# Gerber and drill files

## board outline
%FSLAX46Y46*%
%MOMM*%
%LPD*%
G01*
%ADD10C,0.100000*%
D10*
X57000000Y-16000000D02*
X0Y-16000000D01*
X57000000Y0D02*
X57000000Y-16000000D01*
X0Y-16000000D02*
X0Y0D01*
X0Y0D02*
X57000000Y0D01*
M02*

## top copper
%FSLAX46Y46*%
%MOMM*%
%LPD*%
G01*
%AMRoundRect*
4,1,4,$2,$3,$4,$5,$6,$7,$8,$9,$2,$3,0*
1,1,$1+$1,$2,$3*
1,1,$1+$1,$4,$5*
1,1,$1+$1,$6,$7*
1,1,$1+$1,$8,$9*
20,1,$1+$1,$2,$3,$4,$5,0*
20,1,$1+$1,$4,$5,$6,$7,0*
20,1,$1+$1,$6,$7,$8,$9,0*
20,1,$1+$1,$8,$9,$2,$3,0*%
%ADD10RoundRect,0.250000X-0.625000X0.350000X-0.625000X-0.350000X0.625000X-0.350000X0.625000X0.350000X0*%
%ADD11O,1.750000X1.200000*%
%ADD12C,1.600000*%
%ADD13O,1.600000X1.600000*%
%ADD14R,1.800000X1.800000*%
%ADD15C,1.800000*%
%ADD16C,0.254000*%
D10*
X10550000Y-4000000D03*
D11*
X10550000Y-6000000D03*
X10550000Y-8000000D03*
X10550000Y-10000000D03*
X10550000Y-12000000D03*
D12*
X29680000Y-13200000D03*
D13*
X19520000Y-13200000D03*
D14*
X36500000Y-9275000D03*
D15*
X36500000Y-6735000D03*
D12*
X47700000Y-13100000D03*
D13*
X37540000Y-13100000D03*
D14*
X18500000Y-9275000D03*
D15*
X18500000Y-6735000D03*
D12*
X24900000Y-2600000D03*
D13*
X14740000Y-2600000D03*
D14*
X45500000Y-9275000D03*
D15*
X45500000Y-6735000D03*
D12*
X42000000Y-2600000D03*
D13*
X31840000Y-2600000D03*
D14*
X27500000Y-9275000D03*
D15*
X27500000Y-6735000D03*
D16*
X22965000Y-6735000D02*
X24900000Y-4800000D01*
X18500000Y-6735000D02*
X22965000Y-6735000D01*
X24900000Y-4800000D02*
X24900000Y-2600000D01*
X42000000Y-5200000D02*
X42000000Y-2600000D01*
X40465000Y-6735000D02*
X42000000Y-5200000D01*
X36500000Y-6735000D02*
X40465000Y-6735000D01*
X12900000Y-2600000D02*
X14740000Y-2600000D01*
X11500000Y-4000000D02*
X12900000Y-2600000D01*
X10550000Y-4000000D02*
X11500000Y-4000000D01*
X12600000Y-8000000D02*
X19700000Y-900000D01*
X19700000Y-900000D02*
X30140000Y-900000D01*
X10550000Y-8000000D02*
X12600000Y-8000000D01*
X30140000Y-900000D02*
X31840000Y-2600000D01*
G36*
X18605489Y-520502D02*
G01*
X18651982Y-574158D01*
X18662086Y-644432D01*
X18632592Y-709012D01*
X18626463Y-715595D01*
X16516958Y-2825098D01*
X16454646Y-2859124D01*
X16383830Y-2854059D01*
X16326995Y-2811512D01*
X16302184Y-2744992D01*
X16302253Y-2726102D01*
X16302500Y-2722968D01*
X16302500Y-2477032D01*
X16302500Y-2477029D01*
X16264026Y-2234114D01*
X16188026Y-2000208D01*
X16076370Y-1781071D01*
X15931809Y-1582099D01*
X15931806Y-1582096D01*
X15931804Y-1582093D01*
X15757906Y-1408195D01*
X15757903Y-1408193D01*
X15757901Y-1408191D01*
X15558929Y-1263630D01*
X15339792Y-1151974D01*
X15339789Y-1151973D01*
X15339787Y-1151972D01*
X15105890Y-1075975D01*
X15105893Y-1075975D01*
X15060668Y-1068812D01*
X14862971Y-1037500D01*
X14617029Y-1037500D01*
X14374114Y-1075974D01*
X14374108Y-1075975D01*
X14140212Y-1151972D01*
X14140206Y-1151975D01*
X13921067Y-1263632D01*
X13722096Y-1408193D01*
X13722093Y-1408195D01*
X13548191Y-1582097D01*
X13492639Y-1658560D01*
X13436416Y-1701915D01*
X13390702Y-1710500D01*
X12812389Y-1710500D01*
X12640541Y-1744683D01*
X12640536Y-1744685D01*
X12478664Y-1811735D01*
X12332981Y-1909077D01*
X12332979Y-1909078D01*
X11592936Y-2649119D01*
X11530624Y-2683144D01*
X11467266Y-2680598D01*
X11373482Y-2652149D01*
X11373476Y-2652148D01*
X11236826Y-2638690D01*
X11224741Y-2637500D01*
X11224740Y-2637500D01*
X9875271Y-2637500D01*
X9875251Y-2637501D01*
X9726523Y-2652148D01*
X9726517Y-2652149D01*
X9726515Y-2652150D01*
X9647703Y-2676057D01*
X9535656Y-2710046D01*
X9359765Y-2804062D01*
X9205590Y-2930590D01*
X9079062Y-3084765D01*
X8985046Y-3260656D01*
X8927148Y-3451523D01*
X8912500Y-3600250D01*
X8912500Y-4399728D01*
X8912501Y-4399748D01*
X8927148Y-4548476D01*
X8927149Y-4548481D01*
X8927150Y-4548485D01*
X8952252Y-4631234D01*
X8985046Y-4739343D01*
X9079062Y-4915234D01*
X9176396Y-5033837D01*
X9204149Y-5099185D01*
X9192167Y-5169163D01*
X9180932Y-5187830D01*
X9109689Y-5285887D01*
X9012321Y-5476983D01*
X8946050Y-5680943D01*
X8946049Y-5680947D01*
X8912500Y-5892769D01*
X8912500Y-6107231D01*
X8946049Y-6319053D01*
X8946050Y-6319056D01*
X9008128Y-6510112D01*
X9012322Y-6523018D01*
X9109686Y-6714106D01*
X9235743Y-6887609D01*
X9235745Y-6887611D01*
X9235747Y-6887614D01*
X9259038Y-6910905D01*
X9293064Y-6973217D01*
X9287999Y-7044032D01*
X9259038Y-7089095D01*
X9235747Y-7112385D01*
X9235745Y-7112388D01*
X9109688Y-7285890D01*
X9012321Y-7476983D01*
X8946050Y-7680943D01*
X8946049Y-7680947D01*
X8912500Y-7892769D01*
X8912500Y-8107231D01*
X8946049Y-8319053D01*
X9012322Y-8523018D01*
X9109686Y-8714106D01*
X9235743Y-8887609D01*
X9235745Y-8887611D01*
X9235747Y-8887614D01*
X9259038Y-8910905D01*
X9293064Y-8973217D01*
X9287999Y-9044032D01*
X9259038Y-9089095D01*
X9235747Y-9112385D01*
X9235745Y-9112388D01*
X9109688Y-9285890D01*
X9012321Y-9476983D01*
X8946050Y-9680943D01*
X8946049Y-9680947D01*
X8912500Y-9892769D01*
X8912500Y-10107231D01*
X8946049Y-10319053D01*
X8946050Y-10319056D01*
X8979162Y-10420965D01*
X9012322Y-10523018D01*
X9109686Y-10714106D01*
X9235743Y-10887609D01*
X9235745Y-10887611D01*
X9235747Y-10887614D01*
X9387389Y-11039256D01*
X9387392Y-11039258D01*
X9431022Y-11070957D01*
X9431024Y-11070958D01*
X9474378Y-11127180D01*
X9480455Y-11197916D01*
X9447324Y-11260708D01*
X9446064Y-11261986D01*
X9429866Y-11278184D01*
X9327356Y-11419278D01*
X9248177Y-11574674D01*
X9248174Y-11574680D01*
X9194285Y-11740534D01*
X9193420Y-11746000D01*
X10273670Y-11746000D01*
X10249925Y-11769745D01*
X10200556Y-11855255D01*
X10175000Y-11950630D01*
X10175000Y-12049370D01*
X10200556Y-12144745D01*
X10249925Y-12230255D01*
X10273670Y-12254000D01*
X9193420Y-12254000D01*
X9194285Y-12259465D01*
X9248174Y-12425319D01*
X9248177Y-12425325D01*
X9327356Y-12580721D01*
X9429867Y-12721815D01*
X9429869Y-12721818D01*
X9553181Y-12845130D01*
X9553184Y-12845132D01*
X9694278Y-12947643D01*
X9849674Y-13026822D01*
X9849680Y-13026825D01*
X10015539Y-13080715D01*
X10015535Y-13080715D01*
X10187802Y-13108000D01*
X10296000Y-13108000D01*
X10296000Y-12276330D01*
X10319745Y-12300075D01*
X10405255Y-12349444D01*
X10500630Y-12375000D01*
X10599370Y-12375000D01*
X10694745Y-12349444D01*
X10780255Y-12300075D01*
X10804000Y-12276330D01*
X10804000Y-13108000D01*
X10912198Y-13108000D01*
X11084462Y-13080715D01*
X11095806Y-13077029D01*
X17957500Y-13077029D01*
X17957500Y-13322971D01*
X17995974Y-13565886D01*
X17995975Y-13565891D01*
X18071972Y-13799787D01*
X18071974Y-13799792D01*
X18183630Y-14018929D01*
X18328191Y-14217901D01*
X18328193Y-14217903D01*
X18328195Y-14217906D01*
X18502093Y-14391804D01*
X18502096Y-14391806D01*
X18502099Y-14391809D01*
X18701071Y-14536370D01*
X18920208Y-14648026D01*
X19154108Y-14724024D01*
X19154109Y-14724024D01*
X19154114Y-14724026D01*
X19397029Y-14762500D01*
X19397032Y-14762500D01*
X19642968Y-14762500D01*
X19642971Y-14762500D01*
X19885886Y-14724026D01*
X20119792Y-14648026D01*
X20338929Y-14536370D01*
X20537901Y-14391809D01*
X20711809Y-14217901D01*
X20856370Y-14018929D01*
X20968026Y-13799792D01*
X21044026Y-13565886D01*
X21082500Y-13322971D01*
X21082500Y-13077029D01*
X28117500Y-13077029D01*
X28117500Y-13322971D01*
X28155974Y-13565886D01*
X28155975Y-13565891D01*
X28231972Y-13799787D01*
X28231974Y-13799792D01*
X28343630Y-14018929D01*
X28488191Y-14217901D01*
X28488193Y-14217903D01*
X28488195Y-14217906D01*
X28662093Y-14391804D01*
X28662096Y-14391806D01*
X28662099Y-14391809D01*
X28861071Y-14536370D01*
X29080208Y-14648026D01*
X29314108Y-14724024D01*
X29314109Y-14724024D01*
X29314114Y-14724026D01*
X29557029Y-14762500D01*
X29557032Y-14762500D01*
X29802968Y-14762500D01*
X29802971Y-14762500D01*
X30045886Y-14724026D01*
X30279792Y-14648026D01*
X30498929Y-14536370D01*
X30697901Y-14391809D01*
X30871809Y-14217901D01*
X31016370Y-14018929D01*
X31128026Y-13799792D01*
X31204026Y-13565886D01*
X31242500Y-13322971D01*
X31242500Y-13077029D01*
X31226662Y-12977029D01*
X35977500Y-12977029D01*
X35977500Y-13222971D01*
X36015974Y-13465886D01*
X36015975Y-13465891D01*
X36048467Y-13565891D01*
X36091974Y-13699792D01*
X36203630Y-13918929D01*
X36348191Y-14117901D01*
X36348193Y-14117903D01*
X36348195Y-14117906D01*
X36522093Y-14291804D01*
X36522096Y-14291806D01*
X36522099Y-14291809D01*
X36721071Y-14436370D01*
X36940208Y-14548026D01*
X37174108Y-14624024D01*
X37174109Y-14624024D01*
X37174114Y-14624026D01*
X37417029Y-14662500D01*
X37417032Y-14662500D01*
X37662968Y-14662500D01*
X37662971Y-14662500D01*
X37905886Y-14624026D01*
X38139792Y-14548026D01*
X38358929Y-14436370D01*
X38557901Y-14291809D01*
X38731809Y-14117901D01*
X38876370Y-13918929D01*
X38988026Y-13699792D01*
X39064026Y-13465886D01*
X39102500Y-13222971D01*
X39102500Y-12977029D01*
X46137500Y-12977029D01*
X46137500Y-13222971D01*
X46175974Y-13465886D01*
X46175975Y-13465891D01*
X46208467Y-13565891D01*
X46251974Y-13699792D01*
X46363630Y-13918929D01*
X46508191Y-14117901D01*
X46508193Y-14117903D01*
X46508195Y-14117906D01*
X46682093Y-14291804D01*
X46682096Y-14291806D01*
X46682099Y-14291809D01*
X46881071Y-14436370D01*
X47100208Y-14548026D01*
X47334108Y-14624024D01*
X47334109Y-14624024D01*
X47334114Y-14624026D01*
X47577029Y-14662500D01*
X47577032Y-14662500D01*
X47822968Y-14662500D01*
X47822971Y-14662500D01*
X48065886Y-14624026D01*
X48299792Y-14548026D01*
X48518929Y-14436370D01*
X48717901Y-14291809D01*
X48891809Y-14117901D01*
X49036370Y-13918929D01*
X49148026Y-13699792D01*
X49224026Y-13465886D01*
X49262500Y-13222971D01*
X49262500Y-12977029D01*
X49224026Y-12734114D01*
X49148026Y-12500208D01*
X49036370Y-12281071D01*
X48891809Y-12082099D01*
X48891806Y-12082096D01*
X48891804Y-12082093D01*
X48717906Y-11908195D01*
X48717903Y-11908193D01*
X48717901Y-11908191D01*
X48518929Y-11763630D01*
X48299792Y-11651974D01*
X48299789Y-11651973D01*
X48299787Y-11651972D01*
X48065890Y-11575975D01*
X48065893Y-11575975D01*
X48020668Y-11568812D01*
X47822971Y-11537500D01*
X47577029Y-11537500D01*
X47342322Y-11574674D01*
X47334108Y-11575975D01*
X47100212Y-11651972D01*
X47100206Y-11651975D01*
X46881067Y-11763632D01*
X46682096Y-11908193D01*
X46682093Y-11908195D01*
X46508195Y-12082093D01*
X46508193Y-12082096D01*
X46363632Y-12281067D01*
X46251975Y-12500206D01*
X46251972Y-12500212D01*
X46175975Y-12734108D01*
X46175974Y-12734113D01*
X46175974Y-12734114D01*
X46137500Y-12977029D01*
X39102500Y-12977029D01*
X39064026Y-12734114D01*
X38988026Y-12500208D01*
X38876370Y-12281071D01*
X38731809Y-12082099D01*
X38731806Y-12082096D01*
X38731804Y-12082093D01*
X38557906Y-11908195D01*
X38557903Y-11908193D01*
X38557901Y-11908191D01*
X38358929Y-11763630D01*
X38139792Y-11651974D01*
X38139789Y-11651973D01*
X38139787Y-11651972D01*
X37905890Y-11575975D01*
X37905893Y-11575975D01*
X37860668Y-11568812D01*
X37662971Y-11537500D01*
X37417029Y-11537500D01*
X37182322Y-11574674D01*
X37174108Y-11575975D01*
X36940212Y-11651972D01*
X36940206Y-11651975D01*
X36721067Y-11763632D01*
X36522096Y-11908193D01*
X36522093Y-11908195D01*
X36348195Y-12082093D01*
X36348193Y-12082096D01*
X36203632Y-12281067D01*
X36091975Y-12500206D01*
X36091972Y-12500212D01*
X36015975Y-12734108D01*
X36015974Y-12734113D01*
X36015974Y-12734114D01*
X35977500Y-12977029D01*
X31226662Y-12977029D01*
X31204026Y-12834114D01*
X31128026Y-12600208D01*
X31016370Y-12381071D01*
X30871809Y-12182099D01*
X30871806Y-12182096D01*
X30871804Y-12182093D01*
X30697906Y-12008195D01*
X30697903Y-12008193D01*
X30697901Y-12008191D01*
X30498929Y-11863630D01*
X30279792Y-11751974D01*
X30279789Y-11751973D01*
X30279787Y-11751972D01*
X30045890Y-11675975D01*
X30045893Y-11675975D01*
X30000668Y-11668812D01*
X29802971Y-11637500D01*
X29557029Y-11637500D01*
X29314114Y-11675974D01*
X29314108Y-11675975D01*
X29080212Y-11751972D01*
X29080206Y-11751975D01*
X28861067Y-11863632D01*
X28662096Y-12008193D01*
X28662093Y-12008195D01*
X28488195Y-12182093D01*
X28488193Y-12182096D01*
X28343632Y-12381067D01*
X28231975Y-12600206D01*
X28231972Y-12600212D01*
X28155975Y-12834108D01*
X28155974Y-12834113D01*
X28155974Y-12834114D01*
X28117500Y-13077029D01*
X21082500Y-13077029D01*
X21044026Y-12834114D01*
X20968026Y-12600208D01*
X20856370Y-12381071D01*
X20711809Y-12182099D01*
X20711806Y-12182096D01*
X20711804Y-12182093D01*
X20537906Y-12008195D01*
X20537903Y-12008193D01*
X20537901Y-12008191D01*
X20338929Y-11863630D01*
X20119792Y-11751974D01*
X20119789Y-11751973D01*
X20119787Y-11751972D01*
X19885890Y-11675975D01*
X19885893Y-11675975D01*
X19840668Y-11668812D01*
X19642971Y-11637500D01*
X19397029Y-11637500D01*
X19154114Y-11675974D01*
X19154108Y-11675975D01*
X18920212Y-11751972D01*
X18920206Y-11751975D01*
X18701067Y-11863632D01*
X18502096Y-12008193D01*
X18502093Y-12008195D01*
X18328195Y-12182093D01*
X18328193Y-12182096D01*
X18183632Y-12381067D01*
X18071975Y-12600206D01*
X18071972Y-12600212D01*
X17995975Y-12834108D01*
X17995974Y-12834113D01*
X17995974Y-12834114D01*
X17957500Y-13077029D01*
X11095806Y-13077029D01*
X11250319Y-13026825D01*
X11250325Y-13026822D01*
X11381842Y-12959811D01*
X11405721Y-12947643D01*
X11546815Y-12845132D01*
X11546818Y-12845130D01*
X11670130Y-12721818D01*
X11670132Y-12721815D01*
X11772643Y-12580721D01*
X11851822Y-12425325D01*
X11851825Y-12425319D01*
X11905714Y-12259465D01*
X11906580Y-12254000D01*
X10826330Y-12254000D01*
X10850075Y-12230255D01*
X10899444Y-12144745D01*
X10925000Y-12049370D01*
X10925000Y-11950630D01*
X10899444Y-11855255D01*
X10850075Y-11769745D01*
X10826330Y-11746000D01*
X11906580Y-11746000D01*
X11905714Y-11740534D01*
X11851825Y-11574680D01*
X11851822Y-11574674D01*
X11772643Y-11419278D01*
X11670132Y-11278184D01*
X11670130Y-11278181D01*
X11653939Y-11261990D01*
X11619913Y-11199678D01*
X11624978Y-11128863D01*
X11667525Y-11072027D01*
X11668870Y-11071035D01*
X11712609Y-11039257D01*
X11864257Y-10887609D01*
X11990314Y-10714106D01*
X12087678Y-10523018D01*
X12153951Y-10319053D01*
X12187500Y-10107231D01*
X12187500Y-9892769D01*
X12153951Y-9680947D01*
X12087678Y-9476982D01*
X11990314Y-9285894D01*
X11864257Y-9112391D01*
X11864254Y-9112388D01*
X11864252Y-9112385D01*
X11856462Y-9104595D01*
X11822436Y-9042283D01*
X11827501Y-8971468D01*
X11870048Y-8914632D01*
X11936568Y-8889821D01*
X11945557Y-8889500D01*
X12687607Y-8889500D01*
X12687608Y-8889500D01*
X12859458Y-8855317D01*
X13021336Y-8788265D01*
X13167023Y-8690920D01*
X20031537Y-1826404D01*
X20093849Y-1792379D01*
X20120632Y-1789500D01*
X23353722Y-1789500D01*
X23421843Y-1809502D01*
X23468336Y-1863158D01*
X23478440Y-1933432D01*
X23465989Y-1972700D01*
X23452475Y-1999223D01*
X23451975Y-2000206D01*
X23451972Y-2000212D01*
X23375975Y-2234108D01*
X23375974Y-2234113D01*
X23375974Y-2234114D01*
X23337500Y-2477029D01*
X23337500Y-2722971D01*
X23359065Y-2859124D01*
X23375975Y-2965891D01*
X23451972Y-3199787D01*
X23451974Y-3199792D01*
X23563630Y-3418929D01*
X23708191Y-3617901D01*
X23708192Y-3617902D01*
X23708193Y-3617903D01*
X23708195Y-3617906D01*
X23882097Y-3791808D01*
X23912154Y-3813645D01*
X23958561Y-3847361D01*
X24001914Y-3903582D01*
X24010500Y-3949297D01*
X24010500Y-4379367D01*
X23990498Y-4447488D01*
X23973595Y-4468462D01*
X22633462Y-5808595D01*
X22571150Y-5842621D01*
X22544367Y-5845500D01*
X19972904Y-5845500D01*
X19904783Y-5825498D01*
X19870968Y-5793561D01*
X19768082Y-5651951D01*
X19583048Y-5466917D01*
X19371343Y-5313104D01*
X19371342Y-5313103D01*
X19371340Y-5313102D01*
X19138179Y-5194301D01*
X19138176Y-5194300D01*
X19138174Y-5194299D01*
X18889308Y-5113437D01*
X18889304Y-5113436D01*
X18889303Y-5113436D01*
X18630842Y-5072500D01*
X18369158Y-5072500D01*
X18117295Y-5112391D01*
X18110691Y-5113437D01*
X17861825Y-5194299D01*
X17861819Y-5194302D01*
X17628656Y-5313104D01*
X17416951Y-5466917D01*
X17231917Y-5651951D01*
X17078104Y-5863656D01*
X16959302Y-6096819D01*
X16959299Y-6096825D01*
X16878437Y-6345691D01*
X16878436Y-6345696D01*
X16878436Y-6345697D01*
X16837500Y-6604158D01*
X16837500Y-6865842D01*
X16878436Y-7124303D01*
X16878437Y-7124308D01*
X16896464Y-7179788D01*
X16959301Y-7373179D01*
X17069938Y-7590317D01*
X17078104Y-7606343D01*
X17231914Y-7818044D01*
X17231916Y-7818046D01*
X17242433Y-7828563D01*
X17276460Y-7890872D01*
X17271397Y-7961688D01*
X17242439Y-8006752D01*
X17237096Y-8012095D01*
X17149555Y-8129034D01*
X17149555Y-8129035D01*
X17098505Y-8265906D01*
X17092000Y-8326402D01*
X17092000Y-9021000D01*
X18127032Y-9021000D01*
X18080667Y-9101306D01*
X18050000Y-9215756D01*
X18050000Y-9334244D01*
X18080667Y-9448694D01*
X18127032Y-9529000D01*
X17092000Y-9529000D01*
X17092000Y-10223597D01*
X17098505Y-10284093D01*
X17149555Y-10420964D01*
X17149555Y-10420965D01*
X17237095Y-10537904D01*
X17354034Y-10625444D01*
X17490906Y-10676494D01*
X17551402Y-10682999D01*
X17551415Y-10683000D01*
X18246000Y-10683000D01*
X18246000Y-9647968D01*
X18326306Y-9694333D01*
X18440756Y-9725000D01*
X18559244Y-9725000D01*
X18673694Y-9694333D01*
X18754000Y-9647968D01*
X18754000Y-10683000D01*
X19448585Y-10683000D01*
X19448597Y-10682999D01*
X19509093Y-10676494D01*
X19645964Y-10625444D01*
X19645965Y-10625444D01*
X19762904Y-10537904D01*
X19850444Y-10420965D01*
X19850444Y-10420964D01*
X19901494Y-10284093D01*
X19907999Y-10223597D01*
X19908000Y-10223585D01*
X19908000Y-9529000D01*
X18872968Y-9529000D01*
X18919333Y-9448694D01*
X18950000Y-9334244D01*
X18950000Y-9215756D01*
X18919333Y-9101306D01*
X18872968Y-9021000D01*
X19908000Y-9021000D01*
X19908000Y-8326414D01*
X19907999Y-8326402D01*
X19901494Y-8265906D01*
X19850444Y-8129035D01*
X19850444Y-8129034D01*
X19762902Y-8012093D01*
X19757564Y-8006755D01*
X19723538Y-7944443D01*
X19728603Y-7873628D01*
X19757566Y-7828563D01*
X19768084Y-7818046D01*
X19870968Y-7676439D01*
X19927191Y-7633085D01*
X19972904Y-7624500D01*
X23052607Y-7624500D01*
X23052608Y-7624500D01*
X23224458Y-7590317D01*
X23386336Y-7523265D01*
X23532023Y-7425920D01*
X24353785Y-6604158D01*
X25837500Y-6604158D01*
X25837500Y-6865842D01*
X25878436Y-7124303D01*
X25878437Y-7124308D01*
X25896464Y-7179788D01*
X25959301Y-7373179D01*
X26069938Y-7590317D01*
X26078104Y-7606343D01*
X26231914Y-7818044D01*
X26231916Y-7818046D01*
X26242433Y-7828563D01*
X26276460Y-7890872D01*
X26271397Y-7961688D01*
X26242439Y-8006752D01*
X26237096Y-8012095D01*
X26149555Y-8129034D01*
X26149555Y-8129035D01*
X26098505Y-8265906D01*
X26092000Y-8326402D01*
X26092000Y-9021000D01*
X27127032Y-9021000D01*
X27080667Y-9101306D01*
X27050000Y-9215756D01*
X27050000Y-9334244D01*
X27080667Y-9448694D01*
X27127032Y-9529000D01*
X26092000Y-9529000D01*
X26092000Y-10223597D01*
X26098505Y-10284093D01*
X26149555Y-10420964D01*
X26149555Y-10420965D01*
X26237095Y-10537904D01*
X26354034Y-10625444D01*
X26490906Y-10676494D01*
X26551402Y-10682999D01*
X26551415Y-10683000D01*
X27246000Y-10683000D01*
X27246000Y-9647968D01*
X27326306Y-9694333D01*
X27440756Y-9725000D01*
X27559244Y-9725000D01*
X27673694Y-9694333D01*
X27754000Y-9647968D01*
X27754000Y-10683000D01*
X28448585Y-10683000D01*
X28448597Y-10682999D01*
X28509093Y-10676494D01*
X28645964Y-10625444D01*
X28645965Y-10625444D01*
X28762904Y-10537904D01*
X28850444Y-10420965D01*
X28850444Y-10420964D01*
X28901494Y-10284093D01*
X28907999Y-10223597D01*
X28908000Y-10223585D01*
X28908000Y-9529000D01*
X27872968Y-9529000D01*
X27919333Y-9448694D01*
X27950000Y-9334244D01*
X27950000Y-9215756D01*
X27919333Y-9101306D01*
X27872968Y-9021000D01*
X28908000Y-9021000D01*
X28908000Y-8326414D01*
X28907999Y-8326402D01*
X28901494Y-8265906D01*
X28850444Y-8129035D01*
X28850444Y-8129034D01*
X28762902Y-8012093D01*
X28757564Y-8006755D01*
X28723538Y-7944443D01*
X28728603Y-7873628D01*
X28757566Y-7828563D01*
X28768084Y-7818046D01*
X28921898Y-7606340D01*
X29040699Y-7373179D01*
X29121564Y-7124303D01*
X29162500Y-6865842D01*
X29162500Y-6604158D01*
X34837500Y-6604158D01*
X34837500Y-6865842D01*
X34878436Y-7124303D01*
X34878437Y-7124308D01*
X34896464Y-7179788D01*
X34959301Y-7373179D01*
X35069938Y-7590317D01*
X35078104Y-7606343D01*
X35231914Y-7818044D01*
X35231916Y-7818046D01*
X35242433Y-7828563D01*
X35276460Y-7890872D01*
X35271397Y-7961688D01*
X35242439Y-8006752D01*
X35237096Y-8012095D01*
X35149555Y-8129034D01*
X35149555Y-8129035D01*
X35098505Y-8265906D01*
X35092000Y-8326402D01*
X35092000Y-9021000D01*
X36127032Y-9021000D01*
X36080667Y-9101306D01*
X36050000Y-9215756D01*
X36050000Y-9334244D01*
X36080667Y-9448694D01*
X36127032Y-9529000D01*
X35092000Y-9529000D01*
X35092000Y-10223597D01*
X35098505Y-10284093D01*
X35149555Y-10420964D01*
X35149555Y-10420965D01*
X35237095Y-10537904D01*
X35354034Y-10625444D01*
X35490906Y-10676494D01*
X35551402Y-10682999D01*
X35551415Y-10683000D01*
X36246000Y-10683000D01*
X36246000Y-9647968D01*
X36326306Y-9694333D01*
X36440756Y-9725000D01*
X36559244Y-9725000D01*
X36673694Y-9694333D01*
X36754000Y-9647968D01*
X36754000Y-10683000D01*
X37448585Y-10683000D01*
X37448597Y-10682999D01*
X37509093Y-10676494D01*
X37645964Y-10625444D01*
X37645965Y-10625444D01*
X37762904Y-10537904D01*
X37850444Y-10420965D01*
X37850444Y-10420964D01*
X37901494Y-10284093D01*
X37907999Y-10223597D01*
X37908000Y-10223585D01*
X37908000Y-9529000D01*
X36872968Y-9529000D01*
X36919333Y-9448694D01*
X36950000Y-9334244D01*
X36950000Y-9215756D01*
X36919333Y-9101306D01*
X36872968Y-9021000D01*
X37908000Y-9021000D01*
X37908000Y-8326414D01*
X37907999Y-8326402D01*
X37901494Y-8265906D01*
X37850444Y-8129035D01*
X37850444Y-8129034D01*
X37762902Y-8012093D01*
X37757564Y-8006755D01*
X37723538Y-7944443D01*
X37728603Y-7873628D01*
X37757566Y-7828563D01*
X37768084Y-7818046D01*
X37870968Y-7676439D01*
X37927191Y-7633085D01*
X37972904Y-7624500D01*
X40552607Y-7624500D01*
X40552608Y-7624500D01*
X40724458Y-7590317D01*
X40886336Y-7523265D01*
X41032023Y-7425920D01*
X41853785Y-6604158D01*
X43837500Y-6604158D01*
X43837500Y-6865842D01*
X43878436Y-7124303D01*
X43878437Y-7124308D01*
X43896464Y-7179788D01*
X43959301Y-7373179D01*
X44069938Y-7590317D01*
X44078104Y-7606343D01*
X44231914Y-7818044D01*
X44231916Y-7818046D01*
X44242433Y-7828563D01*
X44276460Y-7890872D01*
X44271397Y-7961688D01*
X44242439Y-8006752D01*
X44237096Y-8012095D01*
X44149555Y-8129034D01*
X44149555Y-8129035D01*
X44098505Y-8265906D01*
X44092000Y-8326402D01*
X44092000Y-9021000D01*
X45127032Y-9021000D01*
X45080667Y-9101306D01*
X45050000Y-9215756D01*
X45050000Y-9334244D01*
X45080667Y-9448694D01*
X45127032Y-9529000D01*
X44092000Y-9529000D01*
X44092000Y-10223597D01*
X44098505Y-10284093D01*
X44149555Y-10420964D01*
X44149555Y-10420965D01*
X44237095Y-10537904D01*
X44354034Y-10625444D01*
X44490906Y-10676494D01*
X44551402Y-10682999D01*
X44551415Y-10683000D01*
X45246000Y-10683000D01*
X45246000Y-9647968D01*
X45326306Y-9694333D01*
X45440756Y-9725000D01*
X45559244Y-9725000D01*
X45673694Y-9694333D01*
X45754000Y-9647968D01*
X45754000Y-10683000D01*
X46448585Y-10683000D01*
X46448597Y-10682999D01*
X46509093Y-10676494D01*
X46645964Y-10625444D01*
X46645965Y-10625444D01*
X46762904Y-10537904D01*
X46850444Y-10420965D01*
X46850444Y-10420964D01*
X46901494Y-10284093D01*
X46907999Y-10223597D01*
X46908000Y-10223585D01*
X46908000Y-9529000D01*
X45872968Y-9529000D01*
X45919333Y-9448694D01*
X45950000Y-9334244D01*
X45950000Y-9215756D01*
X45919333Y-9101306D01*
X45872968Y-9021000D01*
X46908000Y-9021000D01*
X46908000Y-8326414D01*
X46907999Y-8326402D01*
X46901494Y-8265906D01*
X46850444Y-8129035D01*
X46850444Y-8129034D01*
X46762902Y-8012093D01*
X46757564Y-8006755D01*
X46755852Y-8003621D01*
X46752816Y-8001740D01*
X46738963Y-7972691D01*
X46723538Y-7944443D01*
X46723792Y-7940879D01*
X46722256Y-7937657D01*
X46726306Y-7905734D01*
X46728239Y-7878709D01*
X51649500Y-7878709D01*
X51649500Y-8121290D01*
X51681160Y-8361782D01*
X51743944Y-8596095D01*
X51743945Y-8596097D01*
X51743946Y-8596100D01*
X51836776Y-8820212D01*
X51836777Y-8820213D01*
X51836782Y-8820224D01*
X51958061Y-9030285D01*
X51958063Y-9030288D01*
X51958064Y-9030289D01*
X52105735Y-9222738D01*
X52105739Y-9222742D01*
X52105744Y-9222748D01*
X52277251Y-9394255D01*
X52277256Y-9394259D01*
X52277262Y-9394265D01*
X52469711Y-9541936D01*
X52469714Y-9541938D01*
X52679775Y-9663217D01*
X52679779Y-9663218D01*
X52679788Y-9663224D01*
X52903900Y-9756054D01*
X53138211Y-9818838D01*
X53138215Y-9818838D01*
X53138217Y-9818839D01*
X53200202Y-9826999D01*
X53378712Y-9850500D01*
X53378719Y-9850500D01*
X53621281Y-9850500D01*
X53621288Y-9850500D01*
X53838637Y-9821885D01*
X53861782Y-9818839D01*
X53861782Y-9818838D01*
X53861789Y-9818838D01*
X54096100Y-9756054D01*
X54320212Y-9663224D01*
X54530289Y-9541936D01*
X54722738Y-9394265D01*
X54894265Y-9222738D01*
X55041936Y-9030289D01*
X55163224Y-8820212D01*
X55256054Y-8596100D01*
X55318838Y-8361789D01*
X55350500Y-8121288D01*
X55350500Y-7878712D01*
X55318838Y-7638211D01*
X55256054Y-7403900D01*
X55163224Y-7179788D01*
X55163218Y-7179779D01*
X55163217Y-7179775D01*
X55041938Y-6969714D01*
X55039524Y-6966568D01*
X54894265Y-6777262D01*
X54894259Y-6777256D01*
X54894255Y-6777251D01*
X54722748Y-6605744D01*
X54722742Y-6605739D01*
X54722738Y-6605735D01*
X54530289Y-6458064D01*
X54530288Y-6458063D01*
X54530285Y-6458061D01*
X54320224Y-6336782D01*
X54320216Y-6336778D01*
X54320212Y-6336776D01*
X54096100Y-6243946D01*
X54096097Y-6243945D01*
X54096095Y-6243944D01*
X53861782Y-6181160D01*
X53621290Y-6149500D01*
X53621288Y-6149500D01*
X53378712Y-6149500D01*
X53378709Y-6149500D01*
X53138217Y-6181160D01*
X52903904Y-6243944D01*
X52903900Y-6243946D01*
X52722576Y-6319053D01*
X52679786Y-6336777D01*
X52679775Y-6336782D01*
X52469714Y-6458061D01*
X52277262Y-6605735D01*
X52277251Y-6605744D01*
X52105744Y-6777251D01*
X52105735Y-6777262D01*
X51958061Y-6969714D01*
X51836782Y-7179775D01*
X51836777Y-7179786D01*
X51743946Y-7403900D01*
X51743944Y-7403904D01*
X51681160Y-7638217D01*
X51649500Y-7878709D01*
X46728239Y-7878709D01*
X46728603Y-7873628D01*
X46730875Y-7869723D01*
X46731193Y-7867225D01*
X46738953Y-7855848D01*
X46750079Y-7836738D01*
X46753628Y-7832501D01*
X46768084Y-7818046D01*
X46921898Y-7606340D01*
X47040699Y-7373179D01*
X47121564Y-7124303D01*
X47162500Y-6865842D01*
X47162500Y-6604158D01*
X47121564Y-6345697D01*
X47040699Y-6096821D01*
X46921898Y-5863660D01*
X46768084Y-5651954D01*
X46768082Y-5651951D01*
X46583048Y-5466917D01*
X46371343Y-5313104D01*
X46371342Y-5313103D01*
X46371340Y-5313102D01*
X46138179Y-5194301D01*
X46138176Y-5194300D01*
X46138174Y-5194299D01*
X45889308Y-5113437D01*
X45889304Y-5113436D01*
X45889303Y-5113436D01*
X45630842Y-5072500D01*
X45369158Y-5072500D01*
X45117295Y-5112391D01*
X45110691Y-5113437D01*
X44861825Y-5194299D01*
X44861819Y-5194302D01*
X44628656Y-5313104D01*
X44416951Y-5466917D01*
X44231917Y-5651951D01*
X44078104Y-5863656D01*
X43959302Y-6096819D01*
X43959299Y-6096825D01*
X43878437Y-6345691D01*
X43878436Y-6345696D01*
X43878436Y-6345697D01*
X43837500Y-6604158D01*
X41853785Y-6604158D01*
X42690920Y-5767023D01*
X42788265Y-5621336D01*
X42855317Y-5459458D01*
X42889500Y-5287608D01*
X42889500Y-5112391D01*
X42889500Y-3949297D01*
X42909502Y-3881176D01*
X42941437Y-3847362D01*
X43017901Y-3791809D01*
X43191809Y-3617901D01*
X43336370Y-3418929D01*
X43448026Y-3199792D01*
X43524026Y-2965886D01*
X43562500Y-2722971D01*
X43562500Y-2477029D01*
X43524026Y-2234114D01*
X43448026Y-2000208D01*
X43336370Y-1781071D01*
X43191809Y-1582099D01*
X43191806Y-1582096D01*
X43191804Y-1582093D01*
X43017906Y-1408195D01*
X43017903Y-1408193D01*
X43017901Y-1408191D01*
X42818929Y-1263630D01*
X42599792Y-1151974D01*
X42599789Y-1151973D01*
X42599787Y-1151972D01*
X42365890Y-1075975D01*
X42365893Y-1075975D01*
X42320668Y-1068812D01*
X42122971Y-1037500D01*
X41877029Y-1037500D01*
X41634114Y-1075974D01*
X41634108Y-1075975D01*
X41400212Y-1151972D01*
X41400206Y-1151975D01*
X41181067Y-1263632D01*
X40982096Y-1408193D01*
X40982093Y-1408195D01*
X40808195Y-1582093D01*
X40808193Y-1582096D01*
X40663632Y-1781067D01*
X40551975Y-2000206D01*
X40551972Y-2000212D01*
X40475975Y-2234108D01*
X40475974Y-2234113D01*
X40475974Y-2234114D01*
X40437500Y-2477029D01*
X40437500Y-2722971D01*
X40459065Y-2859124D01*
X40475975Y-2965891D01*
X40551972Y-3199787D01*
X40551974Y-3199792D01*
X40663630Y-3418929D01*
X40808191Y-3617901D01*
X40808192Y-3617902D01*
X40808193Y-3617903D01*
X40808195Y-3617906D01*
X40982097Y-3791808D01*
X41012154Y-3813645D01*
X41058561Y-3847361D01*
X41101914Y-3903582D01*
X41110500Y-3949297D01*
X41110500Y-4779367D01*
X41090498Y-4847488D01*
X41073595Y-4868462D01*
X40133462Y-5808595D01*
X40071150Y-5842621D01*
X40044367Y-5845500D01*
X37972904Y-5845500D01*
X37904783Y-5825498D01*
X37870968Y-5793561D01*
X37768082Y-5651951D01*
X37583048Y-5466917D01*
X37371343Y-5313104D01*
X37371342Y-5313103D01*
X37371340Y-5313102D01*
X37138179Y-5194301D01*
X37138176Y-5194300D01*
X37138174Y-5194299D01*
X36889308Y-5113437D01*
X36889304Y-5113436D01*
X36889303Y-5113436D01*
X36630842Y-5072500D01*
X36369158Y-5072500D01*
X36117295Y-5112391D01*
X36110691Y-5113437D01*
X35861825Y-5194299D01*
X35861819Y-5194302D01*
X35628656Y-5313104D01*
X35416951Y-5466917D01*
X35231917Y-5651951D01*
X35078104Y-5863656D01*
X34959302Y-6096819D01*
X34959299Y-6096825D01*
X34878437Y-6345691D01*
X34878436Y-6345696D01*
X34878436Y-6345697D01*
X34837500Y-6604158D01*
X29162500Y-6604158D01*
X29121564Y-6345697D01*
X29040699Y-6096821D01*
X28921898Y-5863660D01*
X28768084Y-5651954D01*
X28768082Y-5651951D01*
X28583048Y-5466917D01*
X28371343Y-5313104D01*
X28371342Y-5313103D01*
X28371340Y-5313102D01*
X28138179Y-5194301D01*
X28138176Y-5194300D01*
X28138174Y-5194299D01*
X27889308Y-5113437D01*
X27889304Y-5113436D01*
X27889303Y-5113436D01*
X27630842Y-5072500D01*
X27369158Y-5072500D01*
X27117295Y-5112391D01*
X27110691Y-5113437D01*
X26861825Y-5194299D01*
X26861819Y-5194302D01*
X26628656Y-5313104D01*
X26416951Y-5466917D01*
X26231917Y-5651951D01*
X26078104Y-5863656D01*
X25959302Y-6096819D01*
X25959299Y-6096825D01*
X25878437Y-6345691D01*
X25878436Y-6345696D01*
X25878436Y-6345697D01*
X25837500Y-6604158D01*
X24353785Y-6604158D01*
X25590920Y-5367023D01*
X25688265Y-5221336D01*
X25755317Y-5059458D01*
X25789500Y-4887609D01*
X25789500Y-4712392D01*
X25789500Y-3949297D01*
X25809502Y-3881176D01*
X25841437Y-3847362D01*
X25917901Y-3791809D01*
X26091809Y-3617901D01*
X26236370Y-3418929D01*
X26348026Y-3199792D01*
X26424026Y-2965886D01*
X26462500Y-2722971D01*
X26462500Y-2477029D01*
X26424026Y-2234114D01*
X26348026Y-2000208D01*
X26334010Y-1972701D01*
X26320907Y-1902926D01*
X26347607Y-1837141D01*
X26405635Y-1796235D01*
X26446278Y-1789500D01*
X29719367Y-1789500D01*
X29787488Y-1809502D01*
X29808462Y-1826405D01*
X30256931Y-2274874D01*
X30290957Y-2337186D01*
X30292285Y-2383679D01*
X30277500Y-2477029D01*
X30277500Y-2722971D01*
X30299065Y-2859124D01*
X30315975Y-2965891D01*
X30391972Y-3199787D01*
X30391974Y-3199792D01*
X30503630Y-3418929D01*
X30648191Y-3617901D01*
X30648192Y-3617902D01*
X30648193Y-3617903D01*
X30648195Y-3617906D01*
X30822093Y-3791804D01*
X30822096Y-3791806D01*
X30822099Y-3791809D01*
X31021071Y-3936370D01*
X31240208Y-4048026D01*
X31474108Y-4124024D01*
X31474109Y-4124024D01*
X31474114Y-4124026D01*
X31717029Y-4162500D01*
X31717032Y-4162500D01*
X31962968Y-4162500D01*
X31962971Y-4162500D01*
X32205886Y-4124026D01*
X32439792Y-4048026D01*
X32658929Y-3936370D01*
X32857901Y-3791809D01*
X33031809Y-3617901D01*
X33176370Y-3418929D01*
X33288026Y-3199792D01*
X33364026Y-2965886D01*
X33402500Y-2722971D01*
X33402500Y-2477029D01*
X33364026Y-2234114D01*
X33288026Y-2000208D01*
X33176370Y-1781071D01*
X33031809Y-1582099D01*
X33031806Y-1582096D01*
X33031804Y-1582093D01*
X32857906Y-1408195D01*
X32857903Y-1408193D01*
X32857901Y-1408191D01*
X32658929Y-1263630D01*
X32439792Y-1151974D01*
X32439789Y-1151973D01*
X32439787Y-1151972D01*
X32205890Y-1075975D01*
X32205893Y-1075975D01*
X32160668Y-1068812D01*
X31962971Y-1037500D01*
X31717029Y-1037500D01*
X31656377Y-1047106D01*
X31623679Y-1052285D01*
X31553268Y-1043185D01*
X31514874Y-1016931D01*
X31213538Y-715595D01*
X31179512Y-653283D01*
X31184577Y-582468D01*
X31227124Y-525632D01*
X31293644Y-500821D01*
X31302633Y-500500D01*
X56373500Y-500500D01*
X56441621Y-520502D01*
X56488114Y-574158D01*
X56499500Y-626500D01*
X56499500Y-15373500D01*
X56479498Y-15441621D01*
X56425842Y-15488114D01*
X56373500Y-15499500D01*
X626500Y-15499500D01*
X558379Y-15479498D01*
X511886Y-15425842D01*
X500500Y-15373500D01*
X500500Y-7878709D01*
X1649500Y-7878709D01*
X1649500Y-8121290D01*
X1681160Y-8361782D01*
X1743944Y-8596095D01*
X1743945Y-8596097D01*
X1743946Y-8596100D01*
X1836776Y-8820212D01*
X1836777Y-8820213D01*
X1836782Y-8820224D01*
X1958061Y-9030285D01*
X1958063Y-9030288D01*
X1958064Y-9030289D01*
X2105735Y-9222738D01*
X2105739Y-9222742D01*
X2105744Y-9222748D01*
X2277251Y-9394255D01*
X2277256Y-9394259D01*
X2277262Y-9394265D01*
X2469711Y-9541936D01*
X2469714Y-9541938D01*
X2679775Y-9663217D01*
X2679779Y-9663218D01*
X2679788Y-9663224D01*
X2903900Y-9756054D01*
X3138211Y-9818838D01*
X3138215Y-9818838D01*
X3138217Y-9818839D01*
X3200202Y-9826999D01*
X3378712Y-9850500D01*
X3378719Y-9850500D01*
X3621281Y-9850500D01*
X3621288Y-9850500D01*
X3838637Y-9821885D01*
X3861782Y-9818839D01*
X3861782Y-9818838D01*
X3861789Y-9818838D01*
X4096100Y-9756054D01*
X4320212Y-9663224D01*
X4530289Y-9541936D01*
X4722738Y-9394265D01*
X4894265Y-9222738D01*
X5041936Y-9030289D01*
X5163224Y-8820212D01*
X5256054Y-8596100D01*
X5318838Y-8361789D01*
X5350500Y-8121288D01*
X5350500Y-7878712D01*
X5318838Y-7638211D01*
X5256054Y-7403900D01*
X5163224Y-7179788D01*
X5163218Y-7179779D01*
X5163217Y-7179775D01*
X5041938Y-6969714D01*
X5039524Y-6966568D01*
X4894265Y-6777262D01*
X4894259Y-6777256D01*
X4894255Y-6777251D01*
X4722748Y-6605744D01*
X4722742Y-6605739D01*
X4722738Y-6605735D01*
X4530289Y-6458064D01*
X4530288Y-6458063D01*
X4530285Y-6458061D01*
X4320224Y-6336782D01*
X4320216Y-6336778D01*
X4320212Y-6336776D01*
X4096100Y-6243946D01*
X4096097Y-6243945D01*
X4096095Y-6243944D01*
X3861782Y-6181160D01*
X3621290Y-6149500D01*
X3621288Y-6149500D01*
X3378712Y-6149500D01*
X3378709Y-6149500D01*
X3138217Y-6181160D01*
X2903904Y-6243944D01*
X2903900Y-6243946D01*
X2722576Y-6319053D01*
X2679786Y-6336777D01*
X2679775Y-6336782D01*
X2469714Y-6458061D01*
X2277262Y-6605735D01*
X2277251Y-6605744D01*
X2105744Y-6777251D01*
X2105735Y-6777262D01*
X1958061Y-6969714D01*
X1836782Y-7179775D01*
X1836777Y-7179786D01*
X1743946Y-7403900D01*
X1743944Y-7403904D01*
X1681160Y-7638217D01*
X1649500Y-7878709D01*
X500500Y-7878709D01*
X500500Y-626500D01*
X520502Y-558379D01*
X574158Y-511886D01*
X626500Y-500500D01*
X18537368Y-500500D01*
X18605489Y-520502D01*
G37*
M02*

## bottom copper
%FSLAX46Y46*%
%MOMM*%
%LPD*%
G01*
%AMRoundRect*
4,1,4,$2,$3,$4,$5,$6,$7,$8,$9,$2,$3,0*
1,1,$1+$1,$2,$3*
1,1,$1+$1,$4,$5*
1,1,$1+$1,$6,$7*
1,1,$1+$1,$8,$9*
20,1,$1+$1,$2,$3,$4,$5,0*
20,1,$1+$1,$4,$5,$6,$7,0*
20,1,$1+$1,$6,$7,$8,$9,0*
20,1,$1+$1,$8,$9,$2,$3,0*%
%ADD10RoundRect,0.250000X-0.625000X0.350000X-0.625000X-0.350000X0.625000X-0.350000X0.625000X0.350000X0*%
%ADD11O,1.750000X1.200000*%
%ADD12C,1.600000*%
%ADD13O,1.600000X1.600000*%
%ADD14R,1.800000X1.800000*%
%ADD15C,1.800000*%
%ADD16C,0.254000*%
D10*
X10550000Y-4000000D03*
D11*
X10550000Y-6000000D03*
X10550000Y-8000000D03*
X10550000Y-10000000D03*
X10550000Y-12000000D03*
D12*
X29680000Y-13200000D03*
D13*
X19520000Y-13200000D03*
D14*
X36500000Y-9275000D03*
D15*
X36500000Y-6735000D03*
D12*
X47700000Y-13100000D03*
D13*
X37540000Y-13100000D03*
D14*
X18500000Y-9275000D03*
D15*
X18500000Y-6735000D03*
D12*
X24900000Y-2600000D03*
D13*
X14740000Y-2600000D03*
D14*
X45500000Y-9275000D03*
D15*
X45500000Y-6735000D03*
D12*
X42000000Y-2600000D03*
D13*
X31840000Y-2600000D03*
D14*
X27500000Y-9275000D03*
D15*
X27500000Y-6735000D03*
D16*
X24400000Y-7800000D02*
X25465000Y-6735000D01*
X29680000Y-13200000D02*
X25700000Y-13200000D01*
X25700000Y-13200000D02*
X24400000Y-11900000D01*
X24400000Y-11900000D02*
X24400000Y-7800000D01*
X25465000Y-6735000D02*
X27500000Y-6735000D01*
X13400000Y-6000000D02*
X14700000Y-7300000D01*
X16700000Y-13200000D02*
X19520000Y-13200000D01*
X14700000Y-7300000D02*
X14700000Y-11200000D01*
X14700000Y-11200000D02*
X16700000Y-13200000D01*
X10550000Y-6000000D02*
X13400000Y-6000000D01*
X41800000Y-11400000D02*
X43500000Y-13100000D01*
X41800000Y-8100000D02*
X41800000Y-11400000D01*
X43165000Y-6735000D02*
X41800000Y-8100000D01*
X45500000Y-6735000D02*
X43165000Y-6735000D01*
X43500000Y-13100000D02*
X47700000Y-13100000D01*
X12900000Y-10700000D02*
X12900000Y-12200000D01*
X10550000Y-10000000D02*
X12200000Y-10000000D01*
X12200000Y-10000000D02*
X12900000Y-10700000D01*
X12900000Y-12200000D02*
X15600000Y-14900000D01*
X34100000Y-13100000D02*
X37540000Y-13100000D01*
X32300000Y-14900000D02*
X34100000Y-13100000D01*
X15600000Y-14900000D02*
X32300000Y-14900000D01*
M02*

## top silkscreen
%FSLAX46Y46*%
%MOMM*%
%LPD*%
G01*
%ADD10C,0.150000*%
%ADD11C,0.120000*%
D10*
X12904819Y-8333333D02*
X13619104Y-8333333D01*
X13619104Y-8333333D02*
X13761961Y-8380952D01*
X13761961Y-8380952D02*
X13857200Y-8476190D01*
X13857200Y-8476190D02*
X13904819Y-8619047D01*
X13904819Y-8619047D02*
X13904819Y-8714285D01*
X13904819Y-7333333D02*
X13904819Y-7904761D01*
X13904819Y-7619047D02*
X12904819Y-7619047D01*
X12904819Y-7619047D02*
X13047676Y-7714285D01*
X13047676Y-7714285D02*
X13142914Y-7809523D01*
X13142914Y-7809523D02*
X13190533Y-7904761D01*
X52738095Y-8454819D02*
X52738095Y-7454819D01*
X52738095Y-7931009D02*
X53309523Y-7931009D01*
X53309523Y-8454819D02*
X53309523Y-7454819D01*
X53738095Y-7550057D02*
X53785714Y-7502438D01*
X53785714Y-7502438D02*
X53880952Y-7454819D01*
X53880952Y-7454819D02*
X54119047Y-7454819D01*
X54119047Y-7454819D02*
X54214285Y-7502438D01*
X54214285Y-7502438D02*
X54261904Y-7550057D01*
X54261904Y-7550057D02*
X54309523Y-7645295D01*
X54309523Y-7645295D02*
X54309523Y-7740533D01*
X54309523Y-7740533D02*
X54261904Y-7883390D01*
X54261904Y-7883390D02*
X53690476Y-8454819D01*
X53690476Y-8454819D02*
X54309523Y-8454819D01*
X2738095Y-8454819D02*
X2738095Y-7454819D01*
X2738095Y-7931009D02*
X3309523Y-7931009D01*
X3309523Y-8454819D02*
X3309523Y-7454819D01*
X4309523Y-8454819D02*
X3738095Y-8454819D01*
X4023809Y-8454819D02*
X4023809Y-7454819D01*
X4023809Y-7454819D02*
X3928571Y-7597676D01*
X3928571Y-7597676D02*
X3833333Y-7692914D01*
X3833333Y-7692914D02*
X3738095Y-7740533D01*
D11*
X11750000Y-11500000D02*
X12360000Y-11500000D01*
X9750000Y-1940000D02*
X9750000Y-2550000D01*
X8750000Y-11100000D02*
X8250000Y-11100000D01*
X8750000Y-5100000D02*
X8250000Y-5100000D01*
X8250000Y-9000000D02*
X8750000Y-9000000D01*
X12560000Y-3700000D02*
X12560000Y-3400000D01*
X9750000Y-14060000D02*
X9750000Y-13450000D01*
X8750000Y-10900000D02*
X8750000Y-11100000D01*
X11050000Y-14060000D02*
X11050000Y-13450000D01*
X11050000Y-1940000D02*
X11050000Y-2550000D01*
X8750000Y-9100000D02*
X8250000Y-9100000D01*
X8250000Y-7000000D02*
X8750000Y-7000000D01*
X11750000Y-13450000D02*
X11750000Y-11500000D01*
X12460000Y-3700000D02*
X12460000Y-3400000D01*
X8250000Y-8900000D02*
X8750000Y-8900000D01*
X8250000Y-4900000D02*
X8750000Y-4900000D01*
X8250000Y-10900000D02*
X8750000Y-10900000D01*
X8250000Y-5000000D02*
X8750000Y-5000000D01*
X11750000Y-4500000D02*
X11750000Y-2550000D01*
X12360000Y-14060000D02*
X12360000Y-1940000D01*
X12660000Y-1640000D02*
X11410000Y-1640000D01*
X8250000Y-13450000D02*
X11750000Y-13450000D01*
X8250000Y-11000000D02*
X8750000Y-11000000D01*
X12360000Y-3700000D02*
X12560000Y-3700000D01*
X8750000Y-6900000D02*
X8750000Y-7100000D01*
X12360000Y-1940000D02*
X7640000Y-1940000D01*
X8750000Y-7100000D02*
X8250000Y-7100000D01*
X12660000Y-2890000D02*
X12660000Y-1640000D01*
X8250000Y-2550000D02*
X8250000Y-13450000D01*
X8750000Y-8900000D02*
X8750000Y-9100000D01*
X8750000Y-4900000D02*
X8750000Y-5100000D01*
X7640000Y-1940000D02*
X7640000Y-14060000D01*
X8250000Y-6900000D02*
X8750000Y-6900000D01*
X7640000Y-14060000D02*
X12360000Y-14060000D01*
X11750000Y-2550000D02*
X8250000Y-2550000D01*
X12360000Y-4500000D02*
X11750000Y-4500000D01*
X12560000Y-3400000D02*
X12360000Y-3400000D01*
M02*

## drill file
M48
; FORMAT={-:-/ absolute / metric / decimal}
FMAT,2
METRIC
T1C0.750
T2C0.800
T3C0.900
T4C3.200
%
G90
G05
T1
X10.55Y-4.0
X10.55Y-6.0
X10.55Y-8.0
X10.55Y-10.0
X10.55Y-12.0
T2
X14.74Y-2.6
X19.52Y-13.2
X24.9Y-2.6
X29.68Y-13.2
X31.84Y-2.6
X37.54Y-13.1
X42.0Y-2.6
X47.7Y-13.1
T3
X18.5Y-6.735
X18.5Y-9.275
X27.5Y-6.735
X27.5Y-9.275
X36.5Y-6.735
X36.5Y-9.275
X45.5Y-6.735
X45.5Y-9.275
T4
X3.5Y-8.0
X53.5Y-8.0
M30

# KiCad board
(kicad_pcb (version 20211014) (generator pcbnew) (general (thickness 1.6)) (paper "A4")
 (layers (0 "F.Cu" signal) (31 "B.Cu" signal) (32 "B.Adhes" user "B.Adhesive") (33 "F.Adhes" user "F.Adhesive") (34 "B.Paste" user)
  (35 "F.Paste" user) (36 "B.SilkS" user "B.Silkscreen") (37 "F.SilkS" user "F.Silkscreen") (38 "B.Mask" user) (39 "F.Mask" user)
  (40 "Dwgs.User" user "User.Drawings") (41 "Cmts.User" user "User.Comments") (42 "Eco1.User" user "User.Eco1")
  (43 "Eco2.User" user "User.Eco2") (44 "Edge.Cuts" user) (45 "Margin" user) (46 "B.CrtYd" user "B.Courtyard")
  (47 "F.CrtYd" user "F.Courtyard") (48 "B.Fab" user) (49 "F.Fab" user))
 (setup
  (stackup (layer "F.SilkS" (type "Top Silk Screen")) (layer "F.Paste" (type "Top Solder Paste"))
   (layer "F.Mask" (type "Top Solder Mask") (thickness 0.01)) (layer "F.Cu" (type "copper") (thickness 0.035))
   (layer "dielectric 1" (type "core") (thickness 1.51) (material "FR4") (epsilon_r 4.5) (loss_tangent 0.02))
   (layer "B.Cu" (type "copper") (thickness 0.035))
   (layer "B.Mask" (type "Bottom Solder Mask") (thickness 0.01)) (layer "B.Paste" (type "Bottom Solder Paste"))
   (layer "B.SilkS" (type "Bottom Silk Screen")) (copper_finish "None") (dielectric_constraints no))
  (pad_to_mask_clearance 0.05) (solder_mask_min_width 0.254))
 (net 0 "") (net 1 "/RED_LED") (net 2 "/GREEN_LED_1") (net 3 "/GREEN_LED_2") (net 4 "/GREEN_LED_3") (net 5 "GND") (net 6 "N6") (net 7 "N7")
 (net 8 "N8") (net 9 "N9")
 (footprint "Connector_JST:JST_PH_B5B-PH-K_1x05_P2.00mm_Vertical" (layer "F.Cu") (at 10.55 4 -90)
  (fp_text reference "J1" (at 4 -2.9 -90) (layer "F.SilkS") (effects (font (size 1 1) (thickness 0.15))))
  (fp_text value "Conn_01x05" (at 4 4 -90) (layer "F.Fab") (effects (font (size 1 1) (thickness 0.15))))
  (fp_line (start 7.5 -1.2) (end 7.5 -1.81) (layer "F.SilkS") (width 0.12))
  (fp_line (start -2.06 0.8) (end -1.45 0.8) (layer "F.SilkS") (width 0.12))
  (fp_line (start 7.1 1.8) (end 7.1 2.3) (layer "F.SilkS") (width 0.12))
  (fp_line (start 1.1 1.8) (end 1.1 2.3) (layer "F.SilkS") (width 0.12))
  (fp_line (start 5 2.3) (end 5 1.8) (layer "F.SilkS") (width 0.12))
  (fp_line (start -0.3 -2.01) (end -0.6 -2.01) (layer "F.SilkS") (width 0.12))
  (fp_line (start 10.06 0.8) (end 9.45 0.8) (layer "F.SilkS") (width 0.12))
  (fp_line (start 6.9 1.8) (end 7.1 1.8) (layer "F.SilkS") (width 0.12))
  (fp_line (start 10.06 -0.5) (end 9.45 -0.5) (layer "F.SilkS") (width 0.12))
  (fp_line (start -2.06 -0.5) (end -1.45 -0.5) (layer "F.SilkS") (width 0.12))
  (fp_line (start 5.1 1.8) (end 5.1 2.3) (layer "F.SilkS") (width 0.12))
  (fp_line (start 3 2.3) (end 3 1.8) (layer "F.SilkS") (width 0.12))
  (fp_line (start 9.45 -1.2) (end 7.5 -1.2) (layer "F.SilkS") (width 0.12))
  (fp_line (start -0.3 -1.91) (end -0.6 -1.91) (layer "F.SilkS") (width 0.12))
  (fp_line (start 4.9 2.3) (end 4.9 1.8) (layer "F.SilkS") (width 0.12))
  (fp_line (start 0.9 2.3) (end 0.9 1.8) (layer "F.SilkS") (width 0.12))
  (fp_line (start 6.9 2.3) (end 6.9 1.8) (layer "F.SilkS") (width 0.12))
  (fp_line (start 1 2.3) (end 1 1.8) (layer "F.SilkS") (width 0.12))
  (fp_line (start 0.5 -1.2) (end -1.45 -1.2) (layer "F.SilkS") (width 0.12))
  (fp_line (start 10.06 -1.81) (end -2.06 -1.81) (layer "F.SilkS") (width 0.12))
  (fp_line (start -2.36 -2.11) (end -2.36 -0.86) (layer "F.SilkS") (width 0.12))
  (fp_line (start 9.45 2.3) (end 9.45 -1.2) (layer "F.SilkS") (width 0.12))
  (fp_line (start 7 2.3) (end 7 1.8) (layer "F.SilkS") (width 0.12))
  (fp_line (start -0.3 -1.81) (end -0.3 -2.01) (layer "F.SilkS") (width 0.12))
  (fp_line (start 2.9 1.8) (end 3.1 1.8) (layer "F.SilkS") (width 0.12))
  (fp_line (start -2.06 -1.81) (end -2.06 2.91) (layer "F.SilkS") (width 0.12))
  (fp_line (start 3.1 1.8) (end 3.1 2.3) (layer "F.SilkS") (width 0.12))
  (fp_line (start -1.11 -2.11) (end -2.36 -2.11) (layer "F.SilkS") (width 0.12))
  (fp_line (start -1.45 2.3) (end 9.45 2.3) (layer "F.SilkS") (width 0.12))
  (fp_line (start 4.9 1.8) (end 5.1 1.8) (layer "F.SilkS") (width 0.12))
  (fp_line (start 0.9 1.8) (end 1.1 1.8) (layer "F.SilkS") (width 0.12))
  (fp_line (start -2.06 2.91) (end 10.06 2.91) (layer "F.SilkS") (width 0.12))
  (fp_line (start 2.9 2.3) (end 2.9 1.8) (layer "F.SilkS") (width 0.12))
  (fp_line (start 10.06 2.91) (end 10.06 -1.81) (layer "F.SilkS") (width 0.12))
  (fp_line (start -1.45 -1.2) (end -1.45 2.3) (layer "F.SilkS") (width 0.12))
  (fp_line (start 0.5 -1.81) (end 0.5 -1.2) (layer "F.SilkS") (width 0.12))
  (fp_line (start -0.6 -2.01) (end -0.6 -1.81) (layer "F.SilkS") (width 0.12))
  (pad "1" thru_hole roundrect (at 0 0 270) (size 1.2 1.75) (drill 0.75) (layers *.Cu *.Mask) (roundrect_rratio 0.208333) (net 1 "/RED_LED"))
  (pad "2" thru_hole oval (at 2 0 270) (size 1.2 1.75) (drill 0.75) (layers *.Cu *.Mask) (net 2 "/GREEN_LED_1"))
  (pad "3" thru_hole oval (at 4 0 270) (size 1.2 1.75) (drill 0.75) (layers *.Cu *.Mask) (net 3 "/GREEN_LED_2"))
  (pad "4" thru_hole oval (at 6 0 270) (size 1.2 1.75) (drill 0.75) (layers *.Cu *.Mask) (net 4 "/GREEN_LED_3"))
  (pad "5" thru_hole oval (at 8 0 270) (size 1.2 1.75) (drill 0.75) (layers *.Cu *.Mask) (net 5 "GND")))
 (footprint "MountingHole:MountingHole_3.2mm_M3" (layer "F.Cu") (at 53.5 8)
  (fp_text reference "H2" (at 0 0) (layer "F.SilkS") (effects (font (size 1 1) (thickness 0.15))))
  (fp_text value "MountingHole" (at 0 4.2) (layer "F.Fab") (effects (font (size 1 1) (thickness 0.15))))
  (pad "" np_thru_hole circle (at 0 0) (size 3.2 3.2) (drill 3.2) (layers *.Cu *.Mask)))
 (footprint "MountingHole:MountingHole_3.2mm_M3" (layer "F.Cu") (at 3.5 8)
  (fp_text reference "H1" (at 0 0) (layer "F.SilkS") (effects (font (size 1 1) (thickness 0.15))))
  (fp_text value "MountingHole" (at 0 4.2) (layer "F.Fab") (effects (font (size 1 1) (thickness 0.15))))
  (pad "" np_thru_hole circle (at 0 0) (size 3.2 3.2) (drill 3.2) (layers *.Cu *.Mask)))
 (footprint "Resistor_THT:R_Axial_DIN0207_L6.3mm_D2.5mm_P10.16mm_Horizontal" (layer "B.Cu") (at 29.68 13.2 180)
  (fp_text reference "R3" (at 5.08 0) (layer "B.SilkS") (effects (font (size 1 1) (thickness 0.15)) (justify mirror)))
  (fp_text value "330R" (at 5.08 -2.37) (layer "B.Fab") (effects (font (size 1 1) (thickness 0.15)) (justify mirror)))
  (pad "1" thru_hole circle (at 0 0 180) (size 1.6 1.6) (drill 0.8) (layers *.Cu *.Mask) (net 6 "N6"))
  (pad "2" thru_hole oval (at 10.16 0 180) (size 1.6 1.6) (drill 0.8) (layers *.Cu *.Mask) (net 2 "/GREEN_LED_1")))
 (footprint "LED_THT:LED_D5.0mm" (layer "B.Cu") (at 36.5 9.275 90)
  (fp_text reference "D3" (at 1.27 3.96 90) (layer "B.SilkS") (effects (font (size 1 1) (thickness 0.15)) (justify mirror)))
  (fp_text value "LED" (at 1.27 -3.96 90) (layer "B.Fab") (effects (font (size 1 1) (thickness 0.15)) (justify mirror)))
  (pad "1" thru_hole rect (at 0 0 90) (size 1.8 1.8) (drill 0.9) (layers *.Cu *.Mask) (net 5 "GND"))
  (pad "2" thru_hole circle (at 2.54 0 90) (size 1.8 1.8) (drill 0.9) (layers *.Cu *.Mask) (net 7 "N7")))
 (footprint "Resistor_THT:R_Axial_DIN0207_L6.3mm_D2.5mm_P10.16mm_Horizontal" (layer "B.Cu") (at 47.7 13.1 180)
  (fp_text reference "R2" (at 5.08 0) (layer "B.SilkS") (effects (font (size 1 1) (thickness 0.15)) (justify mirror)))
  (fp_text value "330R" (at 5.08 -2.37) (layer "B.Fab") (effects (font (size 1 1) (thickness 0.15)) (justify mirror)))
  (pad "1" thru_hole circle (at 0 0 180) (size 1.6 1.6) (drill 0.8) (layers *.Cu *.Mask) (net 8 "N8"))
  (pad "2" thru_hole oval (at 10.16 0 180) (size 1.6 1.6) (drill 0.8) (layers *.Cu *.Mask) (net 4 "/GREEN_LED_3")))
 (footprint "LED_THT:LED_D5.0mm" (layer "B.Cu") (at 18.5 9.275 90)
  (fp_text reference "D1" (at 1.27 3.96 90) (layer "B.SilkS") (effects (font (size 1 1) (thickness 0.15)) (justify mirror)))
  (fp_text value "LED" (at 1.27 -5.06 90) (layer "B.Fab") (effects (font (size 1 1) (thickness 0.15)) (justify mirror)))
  (pad "1" thru_hole rect (at 0 0 90) (size 1.8 1.8) (drill 0.9) (layers *.Cu *.Mask) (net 5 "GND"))
  (pad "2" thru_hole circle (at 2.54 0 90) (size 1.8 1.8) (drill 0.9) (layers *.Cu *.Mask) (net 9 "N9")))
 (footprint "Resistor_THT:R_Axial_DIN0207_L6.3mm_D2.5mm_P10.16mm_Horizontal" (layer "B.Cu") (at 24.9 2.6 180)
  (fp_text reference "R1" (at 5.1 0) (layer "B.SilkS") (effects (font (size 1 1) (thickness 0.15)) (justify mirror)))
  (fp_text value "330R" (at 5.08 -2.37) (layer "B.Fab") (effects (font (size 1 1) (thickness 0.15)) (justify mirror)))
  (pad "1" thru_hole circle (at 0 0 180) (size 1.6 1.6) (drill 0.8) (layers *.Cu *.Mask) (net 9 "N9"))
  (pad "2" thru_hole oval (at 10.16 0 180) (size 1.6 1.6) (drill 0.8) (layers *.Cu *.Mask) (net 1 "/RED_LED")))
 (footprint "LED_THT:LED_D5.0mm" (layer "B.Cu") (at 45.5 9.275 90)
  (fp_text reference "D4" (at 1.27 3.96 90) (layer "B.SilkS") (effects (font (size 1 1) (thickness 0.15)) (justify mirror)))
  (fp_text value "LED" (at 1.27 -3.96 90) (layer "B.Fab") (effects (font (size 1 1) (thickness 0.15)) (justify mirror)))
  (pad "1" thru_hole rect (at 0 0 90) (size 1.8 1.8) (drill 0.9) (layers *.Cu *.Mask) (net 5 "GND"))
  (pad "2" thru_hole circle (at 2.54 0 90) (size 1.8 1.8) (drill 0.9) (layers *.Cu *.Mask) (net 8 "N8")))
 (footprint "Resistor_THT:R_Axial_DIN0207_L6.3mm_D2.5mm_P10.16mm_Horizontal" (layer "B.Cu") (at 42 2.6 180)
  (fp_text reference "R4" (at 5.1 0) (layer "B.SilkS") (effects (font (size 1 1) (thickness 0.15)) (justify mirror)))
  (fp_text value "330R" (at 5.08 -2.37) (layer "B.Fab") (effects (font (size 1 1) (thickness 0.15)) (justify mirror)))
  (pad "1" thru_hole circle (at 0 0 180) (size 1.6 1.6) (drill 0.8) (layers *.Cu *.Mask) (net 7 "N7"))
  (pad "2" thru_hole oval (at 10.16 0 180) (size 1.6 1.6) (drill 0.8) (layers *.Cu *.Mask) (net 3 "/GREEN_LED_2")))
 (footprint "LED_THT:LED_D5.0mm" (layer "B.Cu") (at 27.5 9.275 90)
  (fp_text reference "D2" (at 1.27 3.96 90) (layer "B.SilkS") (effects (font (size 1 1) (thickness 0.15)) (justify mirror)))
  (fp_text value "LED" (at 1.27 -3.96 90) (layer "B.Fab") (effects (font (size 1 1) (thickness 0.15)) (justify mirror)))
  (pad "1" thru_hole rect (at 0 0 90) (size 1.8 1.8) (drill 0.9) (layers *.Cu *.Mask) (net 5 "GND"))
  (pad "2" thru_hole circle (at 2.54 0 90) (size 1.8 1.8) (drill 0.9) (layers *.Cu *.Mask) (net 6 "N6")))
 (gr_line (start 57 16) (end 0 16) (layer "Edge.Cuts") (width 0.1))
 (gr_line (start 57 0) (end 57 16) (layer "Edge.Cuts") (width 0.1))
 (gr_line (start 0 16) (end 0 0) (layer "Edge.Cuts") (width 0.1))
 (gr_line (start 0 0) (end 57 0) (layer "Edge.Cuts") (width 0.1))
 (segment (start 22.965 6.735) (end 24.9 4.8) (width 0.254) (layer "F.Cu") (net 9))
 (segment (start 18.5 6.735) (end 22.965 6.735) (width 0.254) (layer "F.Cu") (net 9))
 (segment (start 24.9 4.8) (end 24.9 2.6) (width 0.254) (layer "F.Cu") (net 9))
 (segment (start 24.4 7.8) (end 25.465 6.735) (width 0.254) (layer "B.Cu") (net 6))
 (segment (start 29.68 13.2) (end 25.7 13.2) (width 0.254) (layer "B.Cu") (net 6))
 (segment (start 25.7 13.2) (end 24.4 11.9) (width 0.254) (layer "B.Cu") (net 6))
 (segment (start 24.4 11.9) (end 24.4 7.8) (width 0.254) (layer "B.Cu") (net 6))
 (segment (start 25.465 6.735) (end 27.5 6.735) (width 0.254) (layer "B.Cu") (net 6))
 (segment (start 42 5.2) (end 42 2.6) (width 0.254) (layer "F.Cu") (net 7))
 (segment (start 40.465 6.735) (end 42 5.2) (width 0.254) (layer "F.Cu") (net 7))
 (segment (start 36.5 6.735) (end 40.465 6.735) (width 0.254) (layer "F.Cu") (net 7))
 (segment (start 12.9 2.6) (end 14.74 2.6) (width 0.254) (layer "F.Cu") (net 1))
 (segment (start 11.5 4) (end 12.9 2.6) (width 0.254) (layer "F.Cu") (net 1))
 (segment (start 10.55 4) (end 11.5 4) (width 0.254) (layer "F.Cu") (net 1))
 (segment (start 13.4 6) (end 14.7 7.3) (width 0.254) (layer "B.Cu") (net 2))
 (segment (start 16.7 13.2) (end 19.52 13.2) (width 0.254) (layer "B.Cu") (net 2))
 (segment (start 14.7 7.3) (end 14.7 11.2) (width 0.254) (layer "B.Cu") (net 2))
 (segment (start 14.7 11.2) (end 16.7 13.2) (width 0.254) (layer "B.Cu") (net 2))
 (segment (start 10.55 6) (end 13.4 6) (width 0.254) (layer "B.Cu") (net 2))
 (segment (start 12.6 8) (end 19.7 0.9) (width 0.254) (layer "F.Cu") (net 3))
 (segment (start 19.7 0.9) (end 30.14 0.9) (width 0.254) (layer "F.Cu") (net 3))
 (segment (start 10.55 8) (end 12.6 8) (width 0.254) (layer "F.Cu") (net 3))
 (segment (start 30.14 0.9) (end 31.84 2.6) (width 0.254) (layer "F.Cu") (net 3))
 (segment (start 41.8 11.4) (end 43.5 13.1) (width 0.254) (layer "B.Cu") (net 8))
 (segment (start 41.8 8.1) (end 41.8 11.4) (width 0.254) (layer "B.Cu") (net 8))
 (segment (start 43.165 6.735) (end 41.8 8.1) (width 0.254) (layer "B.Cu") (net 8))
 (segment (start 45.5 6.735) (end 43.165 6.735) (width 0.254) (layer "B.Cu") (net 8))
 (segment (start 43.5 13.1) (end 47.7 13.1) (width 0.254) (layer "B.Cu") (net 8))
 (segment (start 12.9 10.7) (end 12.9 12.2) (width 0.254) (layer "B.Cu") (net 4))
 (segment (start 10.55 10) (end 12.2 10) (width 0.254) (layer "B.Cu") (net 4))
 (segment (start 12.2 10) (end 12.9 10.7) (width 0.254) (layer "B.Cu") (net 4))
 (segment (start 12.9 12.2) (end 15.6 14.9) (width 0.254) (layer "B.Cu") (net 4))
 (segment (start 34.1 13.1) (end 37.54 13.1) (width 0.254) (layer "B.Cu") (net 4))
 (segment (start 32.3 14.9) (end 34.1 13.1) (width 0.254) (layer "B.Cu") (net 4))
 (segment (start 15.6 14.9) (end 32.3 14.9) (width 0.254) (layer "B.Cu") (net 4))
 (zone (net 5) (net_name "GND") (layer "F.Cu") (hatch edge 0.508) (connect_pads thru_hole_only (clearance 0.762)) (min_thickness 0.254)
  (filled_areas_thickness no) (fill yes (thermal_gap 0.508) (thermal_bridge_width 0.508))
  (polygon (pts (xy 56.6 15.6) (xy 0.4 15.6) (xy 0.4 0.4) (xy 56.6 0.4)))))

